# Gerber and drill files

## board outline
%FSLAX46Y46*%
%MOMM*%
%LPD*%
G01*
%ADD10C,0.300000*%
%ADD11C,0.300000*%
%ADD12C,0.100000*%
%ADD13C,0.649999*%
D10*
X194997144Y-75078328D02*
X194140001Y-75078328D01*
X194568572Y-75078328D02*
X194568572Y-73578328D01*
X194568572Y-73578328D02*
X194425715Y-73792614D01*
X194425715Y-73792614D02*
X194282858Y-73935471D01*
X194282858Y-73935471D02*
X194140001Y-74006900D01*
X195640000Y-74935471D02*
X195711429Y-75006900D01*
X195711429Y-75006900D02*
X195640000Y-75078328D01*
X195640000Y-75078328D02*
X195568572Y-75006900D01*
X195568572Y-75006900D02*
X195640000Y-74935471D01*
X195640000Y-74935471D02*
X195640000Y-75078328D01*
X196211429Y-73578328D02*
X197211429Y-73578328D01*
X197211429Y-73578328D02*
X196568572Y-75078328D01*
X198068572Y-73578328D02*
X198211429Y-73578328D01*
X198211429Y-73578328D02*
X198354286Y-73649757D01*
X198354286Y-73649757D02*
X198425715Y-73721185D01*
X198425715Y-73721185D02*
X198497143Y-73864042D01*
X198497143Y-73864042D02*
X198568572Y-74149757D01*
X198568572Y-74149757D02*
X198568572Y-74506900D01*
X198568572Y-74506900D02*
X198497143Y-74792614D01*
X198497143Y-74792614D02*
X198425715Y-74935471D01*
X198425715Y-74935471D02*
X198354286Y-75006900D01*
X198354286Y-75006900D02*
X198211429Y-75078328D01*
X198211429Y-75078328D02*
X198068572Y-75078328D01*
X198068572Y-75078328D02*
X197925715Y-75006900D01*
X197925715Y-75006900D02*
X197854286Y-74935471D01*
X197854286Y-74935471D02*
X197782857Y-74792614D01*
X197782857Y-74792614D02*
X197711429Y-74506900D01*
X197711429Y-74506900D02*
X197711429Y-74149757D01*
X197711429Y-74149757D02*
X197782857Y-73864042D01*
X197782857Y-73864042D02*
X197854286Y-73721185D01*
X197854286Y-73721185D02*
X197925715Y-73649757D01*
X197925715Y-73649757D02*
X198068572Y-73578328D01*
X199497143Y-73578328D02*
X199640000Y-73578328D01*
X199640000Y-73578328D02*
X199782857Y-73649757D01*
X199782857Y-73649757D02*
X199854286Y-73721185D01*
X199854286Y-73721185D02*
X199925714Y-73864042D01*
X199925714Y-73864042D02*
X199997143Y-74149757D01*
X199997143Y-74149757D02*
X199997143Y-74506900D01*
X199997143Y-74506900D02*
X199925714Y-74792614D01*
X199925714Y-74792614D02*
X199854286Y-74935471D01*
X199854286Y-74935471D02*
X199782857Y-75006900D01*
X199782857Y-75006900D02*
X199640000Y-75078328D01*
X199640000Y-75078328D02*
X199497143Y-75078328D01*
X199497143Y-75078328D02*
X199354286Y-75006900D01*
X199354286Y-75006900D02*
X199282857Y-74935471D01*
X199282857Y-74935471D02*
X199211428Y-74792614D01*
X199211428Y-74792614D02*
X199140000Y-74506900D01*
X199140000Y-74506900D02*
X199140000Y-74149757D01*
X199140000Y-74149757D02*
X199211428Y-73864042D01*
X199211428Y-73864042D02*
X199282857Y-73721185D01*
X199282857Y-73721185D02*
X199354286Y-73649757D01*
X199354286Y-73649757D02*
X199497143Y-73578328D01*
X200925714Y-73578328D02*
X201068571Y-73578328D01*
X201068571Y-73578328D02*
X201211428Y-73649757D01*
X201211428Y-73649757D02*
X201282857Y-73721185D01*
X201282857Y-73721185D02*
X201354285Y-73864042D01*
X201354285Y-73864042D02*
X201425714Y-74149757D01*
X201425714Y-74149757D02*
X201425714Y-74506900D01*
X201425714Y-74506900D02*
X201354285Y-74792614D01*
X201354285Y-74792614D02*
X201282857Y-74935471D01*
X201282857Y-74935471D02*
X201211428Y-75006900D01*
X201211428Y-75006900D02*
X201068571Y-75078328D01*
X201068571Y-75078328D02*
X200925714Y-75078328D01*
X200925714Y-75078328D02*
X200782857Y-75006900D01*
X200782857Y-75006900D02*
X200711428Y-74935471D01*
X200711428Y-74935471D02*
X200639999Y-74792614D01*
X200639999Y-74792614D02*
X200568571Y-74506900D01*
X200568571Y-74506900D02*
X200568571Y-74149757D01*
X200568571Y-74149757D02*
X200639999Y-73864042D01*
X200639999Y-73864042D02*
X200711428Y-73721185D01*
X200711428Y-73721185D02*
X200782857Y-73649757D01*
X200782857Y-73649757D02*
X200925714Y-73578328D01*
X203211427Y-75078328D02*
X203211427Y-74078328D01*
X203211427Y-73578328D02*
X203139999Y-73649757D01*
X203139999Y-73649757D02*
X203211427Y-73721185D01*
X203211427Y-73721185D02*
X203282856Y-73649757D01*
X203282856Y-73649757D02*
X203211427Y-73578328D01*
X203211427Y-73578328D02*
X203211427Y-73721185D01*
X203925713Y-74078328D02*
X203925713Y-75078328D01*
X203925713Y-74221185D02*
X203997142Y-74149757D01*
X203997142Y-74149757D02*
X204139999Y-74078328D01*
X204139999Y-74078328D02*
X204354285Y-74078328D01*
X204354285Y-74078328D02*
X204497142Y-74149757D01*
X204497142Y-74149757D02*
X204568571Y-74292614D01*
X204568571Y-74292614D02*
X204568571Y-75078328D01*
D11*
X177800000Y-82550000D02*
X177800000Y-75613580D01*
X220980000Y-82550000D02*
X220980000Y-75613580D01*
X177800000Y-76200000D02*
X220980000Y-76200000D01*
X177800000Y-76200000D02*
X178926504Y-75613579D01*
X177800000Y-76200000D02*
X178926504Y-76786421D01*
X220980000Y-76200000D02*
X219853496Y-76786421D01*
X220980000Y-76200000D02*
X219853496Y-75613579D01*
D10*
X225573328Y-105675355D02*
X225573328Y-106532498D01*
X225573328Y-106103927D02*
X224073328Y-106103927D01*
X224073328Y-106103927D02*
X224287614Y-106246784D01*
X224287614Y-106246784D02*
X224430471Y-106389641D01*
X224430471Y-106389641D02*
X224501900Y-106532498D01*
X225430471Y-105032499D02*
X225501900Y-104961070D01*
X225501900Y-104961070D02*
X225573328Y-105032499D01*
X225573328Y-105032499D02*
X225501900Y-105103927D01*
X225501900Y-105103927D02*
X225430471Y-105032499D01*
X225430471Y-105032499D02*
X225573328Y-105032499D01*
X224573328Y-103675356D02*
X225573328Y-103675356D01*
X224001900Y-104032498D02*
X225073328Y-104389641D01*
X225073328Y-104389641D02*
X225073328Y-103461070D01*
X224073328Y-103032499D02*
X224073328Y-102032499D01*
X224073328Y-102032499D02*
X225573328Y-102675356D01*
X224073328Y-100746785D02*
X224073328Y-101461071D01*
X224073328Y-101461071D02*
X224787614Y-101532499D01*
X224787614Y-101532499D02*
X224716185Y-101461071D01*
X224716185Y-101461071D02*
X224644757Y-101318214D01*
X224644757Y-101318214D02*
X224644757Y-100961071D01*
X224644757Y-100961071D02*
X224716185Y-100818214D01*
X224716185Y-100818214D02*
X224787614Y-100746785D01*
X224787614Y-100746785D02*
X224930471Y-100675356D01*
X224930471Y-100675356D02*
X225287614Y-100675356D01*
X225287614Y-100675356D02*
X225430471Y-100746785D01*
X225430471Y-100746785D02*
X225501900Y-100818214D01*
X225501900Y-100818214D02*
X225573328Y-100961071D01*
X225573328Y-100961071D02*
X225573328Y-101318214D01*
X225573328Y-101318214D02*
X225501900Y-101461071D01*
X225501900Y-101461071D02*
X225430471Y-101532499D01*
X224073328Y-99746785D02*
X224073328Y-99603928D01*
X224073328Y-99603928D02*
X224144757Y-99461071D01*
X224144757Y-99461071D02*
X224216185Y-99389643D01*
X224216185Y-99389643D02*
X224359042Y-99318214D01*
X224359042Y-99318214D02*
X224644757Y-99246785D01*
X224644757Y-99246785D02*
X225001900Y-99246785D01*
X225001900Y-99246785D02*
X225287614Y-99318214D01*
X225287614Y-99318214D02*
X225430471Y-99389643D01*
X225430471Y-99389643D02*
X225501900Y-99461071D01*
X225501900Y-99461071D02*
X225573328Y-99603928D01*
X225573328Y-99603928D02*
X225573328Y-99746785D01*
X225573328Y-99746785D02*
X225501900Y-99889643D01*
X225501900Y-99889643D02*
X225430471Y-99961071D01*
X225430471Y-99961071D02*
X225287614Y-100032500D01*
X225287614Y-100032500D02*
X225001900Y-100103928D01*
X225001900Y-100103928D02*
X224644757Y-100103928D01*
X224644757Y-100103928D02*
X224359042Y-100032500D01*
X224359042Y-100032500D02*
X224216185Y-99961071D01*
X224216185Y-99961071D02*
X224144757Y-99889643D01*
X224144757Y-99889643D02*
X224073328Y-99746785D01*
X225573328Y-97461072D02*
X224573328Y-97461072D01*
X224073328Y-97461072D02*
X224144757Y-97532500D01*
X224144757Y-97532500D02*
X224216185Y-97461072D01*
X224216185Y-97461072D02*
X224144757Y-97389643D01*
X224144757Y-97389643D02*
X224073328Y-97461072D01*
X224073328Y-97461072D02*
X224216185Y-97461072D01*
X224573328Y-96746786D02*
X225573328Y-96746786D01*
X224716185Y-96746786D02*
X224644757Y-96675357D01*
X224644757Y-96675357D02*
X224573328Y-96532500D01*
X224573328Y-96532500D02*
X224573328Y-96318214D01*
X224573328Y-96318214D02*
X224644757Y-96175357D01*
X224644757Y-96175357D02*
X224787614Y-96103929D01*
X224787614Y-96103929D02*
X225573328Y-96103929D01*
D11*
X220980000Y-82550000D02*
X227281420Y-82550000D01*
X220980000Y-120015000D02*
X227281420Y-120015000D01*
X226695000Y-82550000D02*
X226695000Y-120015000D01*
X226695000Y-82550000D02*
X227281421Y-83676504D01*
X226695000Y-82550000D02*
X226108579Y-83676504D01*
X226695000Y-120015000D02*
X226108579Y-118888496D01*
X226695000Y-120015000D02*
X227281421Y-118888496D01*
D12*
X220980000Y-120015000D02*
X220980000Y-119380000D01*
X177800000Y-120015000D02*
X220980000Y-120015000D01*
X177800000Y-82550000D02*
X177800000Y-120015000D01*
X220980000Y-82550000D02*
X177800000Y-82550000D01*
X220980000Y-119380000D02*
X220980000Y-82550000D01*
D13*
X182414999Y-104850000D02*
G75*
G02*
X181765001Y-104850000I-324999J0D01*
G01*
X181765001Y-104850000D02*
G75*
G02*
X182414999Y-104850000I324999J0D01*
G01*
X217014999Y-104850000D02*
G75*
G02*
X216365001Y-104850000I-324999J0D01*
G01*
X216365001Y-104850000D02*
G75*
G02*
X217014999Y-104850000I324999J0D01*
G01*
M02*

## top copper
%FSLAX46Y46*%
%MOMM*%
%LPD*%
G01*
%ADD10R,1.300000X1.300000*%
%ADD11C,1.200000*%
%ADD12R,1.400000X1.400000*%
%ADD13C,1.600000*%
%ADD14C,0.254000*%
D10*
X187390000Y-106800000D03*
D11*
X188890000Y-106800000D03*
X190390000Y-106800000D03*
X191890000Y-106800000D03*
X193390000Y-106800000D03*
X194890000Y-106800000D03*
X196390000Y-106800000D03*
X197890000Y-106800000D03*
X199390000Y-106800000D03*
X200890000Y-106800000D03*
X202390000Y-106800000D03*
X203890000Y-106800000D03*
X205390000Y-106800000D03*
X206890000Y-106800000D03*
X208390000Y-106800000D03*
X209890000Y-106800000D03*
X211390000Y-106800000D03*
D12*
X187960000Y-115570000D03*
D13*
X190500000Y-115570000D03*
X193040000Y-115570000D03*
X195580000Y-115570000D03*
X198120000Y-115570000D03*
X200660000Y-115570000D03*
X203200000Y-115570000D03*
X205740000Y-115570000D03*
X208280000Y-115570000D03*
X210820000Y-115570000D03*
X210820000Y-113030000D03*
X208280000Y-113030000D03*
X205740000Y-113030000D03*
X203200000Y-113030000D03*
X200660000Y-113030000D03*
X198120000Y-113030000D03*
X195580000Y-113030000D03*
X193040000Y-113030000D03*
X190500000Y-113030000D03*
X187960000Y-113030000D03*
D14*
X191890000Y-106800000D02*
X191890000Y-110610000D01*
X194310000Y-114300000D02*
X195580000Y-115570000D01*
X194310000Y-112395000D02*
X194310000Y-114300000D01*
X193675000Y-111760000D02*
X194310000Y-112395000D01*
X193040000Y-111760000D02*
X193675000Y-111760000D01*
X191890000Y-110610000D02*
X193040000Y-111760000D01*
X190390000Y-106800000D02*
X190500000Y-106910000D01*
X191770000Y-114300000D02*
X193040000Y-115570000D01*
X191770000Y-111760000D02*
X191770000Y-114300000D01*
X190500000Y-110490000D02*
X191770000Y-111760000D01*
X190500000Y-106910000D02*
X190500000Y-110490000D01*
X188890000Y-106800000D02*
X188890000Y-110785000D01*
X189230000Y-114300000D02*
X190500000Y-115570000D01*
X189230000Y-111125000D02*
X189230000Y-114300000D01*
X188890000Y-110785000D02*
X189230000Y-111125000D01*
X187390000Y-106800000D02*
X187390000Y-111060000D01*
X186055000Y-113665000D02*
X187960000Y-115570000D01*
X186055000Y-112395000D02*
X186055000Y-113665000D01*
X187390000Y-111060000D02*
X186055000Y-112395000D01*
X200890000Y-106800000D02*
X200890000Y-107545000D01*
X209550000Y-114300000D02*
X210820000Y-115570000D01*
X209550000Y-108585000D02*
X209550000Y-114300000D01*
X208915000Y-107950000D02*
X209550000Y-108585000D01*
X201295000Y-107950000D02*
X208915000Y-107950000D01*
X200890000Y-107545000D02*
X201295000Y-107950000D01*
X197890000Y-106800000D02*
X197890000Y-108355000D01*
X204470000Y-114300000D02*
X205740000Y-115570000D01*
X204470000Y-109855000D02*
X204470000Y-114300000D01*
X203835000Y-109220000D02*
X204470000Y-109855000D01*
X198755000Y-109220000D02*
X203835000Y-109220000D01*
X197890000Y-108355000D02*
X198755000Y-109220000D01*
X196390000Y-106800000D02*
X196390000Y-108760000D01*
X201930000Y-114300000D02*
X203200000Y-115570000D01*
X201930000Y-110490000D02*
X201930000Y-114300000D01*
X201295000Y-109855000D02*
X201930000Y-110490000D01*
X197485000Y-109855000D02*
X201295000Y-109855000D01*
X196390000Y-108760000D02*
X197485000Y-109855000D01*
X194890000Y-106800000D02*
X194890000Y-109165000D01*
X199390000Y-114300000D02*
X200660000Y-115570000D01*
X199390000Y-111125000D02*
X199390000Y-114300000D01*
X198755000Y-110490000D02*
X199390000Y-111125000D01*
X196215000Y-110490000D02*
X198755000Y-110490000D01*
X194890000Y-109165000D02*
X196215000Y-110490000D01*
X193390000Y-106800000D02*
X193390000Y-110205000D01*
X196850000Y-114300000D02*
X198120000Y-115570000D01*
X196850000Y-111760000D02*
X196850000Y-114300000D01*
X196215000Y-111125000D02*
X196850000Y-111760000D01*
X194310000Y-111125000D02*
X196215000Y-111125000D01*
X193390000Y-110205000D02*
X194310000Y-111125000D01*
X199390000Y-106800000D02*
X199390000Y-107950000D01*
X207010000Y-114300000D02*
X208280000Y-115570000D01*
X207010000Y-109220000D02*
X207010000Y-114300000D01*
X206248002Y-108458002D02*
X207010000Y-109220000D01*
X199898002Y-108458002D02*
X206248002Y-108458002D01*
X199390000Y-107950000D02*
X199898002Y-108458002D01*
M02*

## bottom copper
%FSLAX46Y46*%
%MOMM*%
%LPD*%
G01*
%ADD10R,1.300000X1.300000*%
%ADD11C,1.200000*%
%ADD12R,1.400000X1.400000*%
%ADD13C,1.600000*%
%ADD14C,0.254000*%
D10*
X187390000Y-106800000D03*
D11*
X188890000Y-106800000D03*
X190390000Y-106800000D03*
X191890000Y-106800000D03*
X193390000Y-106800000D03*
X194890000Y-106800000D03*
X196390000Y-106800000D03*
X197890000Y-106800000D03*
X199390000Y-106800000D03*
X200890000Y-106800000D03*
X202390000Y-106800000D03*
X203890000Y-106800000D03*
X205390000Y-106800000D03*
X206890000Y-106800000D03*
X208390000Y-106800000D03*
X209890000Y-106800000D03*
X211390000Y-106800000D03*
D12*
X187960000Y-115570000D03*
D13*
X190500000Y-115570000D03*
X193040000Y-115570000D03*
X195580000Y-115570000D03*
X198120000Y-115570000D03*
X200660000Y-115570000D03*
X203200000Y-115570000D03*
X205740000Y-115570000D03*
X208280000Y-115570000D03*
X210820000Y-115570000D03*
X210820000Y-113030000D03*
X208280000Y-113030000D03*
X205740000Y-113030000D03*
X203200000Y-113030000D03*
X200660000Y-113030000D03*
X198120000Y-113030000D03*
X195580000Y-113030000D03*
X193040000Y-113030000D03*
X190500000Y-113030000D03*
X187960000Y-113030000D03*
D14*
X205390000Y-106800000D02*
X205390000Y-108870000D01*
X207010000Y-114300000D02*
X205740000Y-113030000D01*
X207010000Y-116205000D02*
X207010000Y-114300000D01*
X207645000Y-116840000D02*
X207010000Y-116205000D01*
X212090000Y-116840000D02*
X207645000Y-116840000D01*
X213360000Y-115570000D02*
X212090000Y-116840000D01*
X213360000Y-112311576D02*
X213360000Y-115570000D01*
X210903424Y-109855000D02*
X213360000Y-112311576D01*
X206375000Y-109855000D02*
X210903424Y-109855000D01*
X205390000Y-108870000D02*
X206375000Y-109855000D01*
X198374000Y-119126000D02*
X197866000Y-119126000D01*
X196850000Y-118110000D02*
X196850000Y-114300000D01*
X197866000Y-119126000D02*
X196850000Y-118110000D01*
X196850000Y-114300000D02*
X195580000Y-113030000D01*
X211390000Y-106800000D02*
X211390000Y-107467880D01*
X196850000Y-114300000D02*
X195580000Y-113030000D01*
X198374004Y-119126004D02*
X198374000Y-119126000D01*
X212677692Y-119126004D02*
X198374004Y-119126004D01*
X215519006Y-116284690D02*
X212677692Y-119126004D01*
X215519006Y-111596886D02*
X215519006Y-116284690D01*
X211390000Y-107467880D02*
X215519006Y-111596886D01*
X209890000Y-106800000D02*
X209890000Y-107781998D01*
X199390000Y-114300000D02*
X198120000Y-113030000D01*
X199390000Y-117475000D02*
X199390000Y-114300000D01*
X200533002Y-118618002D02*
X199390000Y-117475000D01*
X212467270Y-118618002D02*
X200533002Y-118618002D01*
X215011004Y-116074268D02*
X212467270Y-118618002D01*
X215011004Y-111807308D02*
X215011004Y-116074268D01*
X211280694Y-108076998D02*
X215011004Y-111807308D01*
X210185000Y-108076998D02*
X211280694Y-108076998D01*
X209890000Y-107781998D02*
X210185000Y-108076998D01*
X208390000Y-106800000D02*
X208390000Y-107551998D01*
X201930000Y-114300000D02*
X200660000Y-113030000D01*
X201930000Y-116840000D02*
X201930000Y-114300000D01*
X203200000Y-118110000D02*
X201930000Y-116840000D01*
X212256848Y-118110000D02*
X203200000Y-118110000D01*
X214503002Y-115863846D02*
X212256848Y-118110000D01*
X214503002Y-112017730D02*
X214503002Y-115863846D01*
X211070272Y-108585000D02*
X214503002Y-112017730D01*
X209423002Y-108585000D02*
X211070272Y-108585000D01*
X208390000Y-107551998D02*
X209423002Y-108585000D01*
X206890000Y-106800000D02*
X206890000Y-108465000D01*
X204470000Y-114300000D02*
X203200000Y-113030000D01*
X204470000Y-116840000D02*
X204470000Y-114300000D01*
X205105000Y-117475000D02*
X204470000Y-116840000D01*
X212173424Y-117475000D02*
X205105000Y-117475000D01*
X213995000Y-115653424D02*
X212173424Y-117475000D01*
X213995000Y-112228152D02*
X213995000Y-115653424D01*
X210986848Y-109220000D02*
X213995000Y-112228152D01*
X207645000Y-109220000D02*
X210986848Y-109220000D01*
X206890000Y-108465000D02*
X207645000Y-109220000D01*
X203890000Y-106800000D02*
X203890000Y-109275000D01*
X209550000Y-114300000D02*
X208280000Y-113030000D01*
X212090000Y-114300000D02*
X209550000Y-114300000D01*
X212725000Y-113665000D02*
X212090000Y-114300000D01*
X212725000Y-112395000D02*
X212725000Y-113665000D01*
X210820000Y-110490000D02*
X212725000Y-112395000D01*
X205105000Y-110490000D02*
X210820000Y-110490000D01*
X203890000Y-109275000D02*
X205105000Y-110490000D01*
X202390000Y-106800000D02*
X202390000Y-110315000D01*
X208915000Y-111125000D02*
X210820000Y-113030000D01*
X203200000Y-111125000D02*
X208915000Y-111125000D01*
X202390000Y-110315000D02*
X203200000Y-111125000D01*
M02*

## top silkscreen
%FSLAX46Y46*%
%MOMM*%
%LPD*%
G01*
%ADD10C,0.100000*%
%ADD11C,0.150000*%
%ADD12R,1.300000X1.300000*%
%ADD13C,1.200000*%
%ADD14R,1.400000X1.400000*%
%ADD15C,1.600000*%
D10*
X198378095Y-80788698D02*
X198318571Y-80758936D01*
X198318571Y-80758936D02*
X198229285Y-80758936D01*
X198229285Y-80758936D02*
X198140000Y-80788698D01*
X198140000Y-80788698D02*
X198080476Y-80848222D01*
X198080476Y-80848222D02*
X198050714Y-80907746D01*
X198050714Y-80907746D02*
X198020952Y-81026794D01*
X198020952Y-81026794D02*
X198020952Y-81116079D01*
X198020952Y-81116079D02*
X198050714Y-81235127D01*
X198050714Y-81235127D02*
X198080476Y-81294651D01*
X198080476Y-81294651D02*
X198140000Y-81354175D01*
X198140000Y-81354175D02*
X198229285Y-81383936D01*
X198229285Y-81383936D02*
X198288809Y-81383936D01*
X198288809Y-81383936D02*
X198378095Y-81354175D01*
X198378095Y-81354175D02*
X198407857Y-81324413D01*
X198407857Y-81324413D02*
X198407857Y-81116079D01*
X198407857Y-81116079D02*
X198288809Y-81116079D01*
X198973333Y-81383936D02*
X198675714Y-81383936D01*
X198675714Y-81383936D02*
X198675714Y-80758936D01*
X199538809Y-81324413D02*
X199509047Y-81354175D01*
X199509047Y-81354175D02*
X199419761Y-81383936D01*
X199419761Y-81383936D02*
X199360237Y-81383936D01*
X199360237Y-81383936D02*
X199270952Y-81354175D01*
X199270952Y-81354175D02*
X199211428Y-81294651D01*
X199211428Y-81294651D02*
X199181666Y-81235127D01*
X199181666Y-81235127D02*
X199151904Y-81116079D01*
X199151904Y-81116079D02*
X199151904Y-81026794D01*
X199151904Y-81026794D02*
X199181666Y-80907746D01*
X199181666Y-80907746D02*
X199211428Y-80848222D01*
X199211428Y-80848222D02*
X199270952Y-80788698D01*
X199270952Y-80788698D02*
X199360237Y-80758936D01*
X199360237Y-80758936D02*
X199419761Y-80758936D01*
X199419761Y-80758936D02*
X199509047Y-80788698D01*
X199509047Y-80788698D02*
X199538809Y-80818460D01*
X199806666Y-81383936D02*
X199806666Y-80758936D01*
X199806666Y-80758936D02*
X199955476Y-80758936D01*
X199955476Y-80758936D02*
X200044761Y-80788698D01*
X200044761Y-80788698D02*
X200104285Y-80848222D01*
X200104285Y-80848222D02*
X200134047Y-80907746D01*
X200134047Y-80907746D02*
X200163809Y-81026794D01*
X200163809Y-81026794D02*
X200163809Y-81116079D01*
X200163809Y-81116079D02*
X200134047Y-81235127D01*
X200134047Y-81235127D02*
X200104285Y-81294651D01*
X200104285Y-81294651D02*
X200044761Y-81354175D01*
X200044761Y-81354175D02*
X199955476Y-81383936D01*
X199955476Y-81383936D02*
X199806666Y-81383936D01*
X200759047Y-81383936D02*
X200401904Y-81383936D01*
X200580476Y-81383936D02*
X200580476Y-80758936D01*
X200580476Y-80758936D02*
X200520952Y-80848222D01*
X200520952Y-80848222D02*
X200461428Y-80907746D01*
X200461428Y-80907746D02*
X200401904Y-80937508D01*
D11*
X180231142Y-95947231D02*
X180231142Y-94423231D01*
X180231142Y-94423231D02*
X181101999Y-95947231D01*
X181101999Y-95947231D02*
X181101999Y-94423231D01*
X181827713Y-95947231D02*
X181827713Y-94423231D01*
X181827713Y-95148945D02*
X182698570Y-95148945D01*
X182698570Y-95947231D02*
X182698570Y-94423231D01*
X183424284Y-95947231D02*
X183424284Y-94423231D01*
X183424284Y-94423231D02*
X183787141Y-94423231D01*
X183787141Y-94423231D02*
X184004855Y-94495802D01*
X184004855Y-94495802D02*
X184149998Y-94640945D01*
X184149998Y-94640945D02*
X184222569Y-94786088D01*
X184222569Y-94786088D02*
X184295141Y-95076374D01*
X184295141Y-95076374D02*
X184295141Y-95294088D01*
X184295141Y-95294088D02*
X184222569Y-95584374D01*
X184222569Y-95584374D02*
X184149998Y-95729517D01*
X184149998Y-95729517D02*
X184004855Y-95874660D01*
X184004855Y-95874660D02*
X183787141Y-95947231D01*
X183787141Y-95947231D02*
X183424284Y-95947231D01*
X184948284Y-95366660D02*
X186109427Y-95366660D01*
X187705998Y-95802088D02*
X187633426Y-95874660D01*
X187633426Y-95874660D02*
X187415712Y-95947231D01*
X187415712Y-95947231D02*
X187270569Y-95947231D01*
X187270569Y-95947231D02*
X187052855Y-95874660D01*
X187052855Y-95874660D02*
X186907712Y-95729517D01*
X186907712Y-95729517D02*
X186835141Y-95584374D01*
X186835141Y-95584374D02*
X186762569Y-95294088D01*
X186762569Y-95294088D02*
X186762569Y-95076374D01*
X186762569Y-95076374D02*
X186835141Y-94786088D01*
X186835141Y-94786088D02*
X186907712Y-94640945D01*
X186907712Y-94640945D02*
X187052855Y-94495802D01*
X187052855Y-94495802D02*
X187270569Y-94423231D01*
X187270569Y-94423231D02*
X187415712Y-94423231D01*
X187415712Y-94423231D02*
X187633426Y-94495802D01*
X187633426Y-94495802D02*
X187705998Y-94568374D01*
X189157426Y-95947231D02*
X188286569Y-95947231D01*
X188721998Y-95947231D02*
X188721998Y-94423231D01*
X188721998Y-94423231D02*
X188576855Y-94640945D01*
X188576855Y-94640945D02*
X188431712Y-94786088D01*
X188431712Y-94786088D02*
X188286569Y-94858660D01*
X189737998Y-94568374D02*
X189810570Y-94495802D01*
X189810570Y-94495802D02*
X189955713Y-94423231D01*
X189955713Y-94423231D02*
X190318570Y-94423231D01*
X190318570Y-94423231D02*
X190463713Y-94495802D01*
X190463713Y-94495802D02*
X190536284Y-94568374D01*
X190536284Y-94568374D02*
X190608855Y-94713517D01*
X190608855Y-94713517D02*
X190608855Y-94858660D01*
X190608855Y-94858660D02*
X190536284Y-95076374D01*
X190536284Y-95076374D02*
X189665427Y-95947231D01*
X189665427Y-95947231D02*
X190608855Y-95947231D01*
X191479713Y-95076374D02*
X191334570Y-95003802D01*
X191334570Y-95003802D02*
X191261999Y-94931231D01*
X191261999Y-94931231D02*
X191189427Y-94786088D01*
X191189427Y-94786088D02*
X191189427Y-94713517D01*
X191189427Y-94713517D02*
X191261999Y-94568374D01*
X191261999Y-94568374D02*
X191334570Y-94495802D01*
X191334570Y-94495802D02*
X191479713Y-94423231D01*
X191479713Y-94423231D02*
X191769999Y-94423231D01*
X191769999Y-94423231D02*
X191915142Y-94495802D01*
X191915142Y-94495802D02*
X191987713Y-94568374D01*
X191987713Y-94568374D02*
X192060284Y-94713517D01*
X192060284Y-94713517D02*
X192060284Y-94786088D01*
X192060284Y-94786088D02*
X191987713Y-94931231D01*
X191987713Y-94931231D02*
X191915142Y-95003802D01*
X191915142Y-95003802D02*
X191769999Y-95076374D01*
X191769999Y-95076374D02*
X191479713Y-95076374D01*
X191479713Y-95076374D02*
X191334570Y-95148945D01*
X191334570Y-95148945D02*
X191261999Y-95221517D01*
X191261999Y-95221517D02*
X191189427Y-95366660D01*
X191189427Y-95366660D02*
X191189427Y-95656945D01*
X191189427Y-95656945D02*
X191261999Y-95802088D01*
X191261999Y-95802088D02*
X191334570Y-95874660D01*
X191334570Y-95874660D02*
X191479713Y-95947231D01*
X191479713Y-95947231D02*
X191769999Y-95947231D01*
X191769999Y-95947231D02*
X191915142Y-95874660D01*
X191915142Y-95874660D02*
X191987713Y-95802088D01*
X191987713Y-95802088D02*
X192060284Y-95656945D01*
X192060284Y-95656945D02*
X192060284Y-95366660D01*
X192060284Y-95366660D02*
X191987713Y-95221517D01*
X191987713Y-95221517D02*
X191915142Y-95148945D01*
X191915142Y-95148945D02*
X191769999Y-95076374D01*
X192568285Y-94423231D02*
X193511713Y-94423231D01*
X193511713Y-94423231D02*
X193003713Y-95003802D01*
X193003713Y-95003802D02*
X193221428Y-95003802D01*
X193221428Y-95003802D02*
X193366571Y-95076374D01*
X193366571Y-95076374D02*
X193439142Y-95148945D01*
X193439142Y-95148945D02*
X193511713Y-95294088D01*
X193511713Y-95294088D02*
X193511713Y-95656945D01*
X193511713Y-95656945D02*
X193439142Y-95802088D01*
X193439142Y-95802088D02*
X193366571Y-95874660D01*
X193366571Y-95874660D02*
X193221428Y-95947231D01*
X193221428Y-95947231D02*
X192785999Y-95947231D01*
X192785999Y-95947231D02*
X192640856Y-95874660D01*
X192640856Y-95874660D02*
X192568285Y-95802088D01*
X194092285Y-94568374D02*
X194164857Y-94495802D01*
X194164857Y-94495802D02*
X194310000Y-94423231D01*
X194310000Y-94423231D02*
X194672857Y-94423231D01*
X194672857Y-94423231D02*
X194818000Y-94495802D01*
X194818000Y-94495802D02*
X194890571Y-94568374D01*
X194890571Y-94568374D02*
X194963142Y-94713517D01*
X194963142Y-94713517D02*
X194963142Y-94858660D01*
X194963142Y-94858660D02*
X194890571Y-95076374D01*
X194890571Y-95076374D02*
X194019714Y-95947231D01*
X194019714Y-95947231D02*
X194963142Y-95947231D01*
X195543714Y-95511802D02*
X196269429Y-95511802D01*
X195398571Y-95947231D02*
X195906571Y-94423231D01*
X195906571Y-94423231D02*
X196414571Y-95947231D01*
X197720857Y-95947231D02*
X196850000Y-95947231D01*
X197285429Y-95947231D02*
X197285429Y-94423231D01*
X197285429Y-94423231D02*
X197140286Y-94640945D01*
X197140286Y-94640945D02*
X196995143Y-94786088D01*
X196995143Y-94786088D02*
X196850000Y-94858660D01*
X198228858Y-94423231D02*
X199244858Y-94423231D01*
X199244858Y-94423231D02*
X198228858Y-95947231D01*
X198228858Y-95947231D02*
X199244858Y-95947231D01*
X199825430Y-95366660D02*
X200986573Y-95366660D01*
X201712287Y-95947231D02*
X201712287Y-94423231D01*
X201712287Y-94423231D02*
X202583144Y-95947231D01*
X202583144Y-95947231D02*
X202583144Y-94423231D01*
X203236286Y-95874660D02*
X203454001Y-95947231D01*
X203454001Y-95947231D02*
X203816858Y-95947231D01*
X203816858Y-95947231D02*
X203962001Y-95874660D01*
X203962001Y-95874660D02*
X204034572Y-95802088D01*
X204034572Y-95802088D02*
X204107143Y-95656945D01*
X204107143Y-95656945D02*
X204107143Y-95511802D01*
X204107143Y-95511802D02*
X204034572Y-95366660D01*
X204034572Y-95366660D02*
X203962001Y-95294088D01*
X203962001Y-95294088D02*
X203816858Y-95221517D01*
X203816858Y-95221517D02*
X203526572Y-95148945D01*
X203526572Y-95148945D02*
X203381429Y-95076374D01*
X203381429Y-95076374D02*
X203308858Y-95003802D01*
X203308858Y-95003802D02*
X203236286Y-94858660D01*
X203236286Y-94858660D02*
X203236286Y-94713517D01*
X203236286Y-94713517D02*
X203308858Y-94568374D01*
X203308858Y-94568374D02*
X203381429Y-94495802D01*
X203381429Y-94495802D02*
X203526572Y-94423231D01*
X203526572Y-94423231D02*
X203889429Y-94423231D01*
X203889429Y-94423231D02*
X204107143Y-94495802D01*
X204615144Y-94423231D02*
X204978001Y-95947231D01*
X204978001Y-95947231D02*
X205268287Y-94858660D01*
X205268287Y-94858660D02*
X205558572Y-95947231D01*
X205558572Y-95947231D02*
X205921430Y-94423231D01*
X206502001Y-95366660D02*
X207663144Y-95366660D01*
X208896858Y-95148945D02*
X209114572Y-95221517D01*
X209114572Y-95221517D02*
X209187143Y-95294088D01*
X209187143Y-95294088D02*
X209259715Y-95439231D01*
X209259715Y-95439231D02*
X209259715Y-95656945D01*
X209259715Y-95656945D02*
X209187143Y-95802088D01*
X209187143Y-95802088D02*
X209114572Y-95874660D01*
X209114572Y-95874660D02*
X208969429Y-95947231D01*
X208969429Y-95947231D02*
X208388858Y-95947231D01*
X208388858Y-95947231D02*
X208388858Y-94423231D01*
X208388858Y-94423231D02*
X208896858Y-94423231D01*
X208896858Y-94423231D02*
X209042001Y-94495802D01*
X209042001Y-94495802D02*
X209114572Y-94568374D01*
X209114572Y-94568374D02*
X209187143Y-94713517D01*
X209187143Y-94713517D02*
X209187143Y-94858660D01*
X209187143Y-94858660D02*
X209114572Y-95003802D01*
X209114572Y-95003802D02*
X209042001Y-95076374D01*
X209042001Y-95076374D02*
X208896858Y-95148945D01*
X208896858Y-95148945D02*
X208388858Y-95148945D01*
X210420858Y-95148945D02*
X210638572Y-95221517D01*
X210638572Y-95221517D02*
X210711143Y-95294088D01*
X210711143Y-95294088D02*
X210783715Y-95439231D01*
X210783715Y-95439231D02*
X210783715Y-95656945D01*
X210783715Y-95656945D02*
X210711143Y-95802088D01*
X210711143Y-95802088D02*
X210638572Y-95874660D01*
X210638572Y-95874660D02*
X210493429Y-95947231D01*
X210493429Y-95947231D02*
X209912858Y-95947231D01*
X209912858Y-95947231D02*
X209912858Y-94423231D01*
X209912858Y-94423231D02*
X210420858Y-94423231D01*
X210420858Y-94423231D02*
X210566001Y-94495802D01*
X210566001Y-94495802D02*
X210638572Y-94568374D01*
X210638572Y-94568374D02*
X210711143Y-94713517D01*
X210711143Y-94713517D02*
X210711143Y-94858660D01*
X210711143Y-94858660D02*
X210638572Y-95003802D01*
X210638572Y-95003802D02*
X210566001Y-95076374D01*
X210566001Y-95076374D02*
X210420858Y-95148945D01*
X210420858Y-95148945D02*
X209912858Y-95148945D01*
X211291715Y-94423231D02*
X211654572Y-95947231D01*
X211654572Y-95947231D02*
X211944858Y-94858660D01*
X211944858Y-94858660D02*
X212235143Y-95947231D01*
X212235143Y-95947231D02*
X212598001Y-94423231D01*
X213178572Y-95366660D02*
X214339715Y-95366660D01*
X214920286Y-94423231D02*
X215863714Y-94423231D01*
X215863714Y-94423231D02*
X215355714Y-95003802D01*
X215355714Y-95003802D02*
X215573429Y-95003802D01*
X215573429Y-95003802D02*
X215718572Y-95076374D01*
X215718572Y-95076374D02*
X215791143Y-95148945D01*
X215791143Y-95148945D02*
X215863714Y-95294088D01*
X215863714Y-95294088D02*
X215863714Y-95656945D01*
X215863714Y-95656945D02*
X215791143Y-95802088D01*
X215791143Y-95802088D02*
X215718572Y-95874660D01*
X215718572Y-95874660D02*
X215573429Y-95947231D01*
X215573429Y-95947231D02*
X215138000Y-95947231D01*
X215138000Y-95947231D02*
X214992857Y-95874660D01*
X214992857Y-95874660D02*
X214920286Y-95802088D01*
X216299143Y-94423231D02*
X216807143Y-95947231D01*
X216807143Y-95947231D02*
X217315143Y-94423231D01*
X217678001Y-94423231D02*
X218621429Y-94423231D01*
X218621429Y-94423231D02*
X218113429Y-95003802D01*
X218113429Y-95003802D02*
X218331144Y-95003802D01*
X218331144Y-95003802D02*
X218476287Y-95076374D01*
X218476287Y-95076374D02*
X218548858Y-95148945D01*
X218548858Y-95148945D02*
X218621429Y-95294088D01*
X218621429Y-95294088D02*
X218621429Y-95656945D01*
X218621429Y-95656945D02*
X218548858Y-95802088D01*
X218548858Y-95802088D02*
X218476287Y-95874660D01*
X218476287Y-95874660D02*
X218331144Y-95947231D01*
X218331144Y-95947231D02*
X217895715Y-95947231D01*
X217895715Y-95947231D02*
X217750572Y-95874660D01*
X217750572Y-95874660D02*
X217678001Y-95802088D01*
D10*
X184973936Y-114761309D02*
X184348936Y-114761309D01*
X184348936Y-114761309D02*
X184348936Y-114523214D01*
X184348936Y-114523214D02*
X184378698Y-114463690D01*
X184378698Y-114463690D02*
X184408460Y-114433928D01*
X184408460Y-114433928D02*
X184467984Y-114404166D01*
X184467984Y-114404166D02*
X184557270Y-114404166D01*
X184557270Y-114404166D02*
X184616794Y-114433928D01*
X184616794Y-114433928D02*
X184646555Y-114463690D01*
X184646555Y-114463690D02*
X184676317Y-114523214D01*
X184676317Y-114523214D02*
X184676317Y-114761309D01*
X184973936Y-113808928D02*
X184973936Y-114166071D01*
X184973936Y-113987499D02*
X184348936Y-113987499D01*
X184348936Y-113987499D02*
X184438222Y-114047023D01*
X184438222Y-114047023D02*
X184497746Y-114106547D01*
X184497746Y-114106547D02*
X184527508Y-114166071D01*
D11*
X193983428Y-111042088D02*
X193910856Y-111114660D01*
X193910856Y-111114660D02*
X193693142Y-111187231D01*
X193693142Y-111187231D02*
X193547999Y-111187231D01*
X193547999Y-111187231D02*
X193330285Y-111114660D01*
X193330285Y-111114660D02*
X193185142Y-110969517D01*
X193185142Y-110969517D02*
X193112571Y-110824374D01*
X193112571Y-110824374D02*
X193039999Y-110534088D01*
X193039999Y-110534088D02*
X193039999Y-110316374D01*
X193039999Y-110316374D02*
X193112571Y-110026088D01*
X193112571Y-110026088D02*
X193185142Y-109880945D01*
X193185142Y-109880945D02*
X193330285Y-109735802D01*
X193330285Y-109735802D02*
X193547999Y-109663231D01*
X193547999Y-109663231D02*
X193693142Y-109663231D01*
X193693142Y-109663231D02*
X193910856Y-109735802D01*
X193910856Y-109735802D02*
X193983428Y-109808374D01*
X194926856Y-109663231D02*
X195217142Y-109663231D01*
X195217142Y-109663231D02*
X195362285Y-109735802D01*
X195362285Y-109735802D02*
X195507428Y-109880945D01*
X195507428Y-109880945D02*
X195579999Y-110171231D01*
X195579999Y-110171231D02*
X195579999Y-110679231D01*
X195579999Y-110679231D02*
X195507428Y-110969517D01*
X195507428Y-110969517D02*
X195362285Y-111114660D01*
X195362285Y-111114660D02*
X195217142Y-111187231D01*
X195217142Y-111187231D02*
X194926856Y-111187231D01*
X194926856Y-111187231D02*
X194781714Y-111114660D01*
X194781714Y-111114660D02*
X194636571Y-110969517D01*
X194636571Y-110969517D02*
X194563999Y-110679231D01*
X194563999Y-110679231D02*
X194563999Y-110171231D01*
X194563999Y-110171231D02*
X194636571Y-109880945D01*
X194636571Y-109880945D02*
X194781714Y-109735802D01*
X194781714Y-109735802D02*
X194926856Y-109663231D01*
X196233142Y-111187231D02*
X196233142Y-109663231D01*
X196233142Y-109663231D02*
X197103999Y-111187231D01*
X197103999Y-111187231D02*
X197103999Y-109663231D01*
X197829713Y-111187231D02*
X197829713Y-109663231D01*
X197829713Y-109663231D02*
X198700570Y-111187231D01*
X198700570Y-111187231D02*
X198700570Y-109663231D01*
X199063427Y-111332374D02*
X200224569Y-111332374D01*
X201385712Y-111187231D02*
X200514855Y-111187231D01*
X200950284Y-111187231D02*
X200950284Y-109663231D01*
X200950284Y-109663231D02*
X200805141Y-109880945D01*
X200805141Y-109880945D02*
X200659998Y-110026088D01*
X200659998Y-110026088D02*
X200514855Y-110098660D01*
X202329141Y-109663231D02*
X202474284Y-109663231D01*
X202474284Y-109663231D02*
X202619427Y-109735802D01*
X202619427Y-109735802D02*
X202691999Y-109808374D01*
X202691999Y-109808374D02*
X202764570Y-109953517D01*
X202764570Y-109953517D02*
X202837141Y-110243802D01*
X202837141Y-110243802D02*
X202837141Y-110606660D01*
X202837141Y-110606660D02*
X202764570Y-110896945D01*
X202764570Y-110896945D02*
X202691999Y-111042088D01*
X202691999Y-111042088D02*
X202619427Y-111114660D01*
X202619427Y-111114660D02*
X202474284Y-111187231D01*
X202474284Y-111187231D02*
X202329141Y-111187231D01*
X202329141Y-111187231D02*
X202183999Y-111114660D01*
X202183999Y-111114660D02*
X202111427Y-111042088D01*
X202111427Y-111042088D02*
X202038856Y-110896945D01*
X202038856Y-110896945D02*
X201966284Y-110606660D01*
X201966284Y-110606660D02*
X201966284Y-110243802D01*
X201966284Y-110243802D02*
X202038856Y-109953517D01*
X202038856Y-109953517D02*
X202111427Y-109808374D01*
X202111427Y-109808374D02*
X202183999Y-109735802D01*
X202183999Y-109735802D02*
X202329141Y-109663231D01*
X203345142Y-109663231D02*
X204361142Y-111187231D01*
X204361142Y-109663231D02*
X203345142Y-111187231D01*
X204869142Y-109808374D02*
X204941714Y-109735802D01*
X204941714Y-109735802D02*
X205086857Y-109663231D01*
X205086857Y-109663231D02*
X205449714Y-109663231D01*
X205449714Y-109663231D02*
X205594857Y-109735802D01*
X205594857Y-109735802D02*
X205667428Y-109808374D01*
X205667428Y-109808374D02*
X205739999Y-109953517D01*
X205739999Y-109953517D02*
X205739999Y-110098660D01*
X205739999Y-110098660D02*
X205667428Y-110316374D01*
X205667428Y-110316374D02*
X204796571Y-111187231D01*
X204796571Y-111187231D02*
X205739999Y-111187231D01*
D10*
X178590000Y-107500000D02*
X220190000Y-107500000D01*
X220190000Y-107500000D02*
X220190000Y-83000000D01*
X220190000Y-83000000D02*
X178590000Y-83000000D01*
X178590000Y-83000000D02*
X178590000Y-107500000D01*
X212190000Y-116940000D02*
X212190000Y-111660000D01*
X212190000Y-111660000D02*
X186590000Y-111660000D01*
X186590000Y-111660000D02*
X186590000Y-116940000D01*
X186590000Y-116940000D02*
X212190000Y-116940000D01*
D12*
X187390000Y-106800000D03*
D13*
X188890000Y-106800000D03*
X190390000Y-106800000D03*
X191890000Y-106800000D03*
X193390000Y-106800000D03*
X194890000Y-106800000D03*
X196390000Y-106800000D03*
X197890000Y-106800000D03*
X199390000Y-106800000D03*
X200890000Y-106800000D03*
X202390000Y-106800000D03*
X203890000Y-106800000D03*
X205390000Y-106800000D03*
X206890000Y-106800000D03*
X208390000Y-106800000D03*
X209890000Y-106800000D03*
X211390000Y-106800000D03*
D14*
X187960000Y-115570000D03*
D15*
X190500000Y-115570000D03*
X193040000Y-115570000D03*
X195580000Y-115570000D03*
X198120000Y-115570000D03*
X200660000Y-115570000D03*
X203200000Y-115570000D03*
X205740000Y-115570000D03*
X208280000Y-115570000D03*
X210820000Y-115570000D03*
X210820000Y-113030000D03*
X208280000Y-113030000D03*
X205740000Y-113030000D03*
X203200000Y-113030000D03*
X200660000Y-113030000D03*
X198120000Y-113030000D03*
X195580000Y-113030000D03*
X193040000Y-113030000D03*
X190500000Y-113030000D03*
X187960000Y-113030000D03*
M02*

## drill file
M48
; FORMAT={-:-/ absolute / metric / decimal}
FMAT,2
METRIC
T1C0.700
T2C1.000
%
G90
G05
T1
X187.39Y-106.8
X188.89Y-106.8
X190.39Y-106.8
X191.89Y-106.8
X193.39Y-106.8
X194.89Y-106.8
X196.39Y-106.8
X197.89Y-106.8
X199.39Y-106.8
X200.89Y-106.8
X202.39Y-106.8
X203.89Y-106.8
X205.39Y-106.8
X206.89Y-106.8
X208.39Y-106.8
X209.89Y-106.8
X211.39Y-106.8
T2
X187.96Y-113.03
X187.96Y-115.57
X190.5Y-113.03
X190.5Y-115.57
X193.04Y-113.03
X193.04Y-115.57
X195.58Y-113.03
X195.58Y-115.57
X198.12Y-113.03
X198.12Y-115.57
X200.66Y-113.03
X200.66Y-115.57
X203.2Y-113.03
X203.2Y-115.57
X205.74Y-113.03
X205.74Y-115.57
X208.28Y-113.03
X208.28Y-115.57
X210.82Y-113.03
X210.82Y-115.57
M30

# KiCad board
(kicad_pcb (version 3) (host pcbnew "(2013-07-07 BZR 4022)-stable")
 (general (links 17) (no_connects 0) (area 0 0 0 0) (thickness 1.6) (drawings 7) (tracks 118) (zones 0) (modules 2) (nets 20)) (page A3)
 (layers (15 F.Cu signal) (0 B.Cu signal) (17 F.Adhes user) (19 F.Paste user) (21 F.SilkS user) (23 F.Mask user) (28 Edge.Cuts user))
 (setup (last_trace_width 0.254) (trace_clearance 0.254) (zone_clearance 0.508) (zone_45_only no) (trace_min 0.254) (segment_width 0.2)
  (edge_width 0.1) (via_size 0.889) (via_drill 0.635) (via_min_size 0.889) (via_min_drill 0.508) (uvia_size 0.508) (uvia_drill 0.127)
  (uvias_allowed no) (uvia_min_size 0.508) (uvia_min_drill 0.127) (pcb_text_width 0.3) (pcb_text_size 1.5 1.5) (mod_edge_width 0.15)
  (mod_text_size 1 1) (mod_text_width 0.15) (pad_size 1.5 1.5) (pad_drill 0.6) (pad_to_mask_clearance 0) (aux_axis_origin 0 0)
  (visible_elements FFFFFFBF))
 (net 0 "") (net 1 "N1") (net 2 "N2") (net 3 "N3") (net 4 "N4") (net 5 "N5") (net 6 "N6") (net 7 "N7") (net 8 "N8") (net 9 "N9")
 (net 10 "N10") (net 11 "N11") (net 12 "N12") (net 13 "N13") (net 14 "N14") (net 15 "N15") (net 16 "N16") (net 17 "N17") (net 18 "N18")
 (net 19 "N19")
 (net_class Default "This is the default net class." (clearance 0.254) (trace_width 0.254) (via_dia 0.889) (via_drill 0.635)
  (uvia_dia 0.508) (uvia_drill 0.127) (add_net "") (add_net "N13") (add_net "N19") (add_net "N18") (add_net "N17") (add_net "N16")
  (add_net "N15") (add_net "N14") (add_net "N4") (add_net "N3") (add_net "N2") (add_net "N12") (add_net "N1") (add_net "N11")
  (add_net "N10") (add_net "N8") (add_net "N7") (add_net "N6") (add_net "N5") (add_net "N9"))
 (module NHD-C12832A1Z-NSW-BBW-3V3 (layer F.Cu) (at 199.39 95.25)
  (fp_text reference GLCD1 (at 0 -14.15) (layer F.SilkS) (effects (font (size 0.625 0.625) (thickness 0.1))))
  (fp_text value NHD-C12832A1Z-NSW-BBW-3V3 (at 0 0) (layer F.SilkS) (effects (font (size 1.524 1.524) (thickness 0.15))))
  (fp_line (start -20.8 12.25) (end 20.8 12.25) (layer F.SilkS) (width 0.1))
  (fp_line (start 20.8 12.25) (end 20.8 -12.25) (layer F.SilkS) (width 0.1))
  (fp_line (start 20.8 -12.25) (end -20.8 -12.25) (layer F.SilkS) (width 0.1))
  (fp_line (start -20.8 -12.25) (end -20.8 12.25) (layer F.SilkS) (width 0.1))
  (fp_circle (center -17.3 9.6) (end -16.840381 10.059619) (layer Edge.Cuts))
  (fp_circle (center 17.3 9.6) (end 17.759619 10.059619) (layer Edge.Cuts))
  (pad 1 thru_hole rect (at -12 11.55) (size 1.3 1.3) (drill 0.7) (layers *.Cu *.Mask F.SilkS) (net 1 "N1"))
  (pad 2 thru_hole circle (at -10.5 11.55) (size 1.2 1.2) (drill 0.7) (layers *.Cu *.Mask F.SilkS) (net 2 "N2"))
  (pad 3 thru_hole circle (at -9 11.55) (size 1.2 1.2) (drill 0.7) (layers *.Cu *.Mask F.SilkS) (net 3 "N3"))
  (pad 4 thru_hole circle (at -7.5 11.55) (size 1.2 1.2) (drill 0.7) (layers *.Cu *.Mask F.SilkS) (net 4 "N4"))
  (pad 5 thru_hole circle (at -6 11.55) (size 1.2 1.2) (drill 0.7) (layers *.Cu *.Mask F.SilkS) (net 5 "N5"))
  (pad 6 thru_hole circle (at -4.5 11.55) (size 1.2 1.2) (drill 0.7) (layers *.Cu *.Mask F.SilkS) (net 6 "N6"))
  (pad 7 thru_hole circle (at -3 11.55) (size 1.2 1.2) (drill 0.7) (layers *.Cu *.Mask F.SilkS) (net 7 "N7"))
  (pad 8 thru_hole circle (at -1.5 11.55) (size 1.2 1.2) (drill 0.7) (layers *.Cu *.Mask F.SilkS) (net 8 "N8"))
  (pad 9 thru_hole circle (at 0 11.55) (size 1.2 1.2) (drill 0.7) (layers *.Cu *.Mask F.SilkS) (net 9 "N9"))
  (pad 10 thru_hole circle (at 1.5 11.55) (size 1.2 1.2) (drill 0.7) (layers *.Cu *.Mask F.SilkS) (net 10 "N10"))
  (pad 11 thru_hole circle (at 3 11.55) (size 1.2 1.2) (drill 0.7) (layers *.Cu *.Mask F.SilkS) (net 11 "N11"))
  (pad 12 thru_hole circle (at 4.5 11.55) (size 1.2 1.2) (drill 0.7) (layers *.Cu *.Mask F.SilkS) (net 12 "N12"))
  (pad 13 thru_hole circle (at 6 11.55) (size 1.2 1.2) (drill 0.7) (layers *.Cu *.Mask F.SilkS) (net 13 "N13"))
  (pad 14 thru_hole circle (at 7.5 11.55) (size 1.2 1.2) (drill 0.7) (layers *.Cu *.Mask F.SilkS) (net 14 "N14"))
  (pad 15 thru_hole circle (at 9 11.55) (size 1.2 1.2) (drill 0.7) (layers *.Cu *.Mask F.SilkS) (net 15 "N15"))
  (pad 16 thru_hole circle (at 10.5 11.55) (size 1.2 1.2) (drill 0.7) (layers *.Cu *.Mask F.SilkS) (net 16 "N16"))
  (pad 17 thru_hole circle (at 12 11.55) (size 1.2 1.2) (drill 0.7) (layers *.Cu *.Mask F.SilkS) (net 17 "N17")))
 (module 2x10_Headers (layer F.Cu) (at 199.39 114.3 90)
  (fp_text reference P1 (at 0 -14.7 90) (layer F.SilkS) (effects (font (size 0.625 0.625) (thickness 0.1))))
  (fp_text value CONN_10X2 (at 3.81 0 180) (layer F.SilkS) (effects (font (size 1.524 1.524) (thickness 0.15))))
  (fp_line (start -2.64 12.8) (end 2.64 12.8) (layer F.SilkS) (width 0.1))
  (fp_line (start 2.64 12.8) (end 2.64 -12.8) (layer F.SilkS) (width 0.1))
  (fp_line (start 2.64 -12.8) (end -2.64 -12.8) (layer F.SilkS) (width 0.1))
  (fp_line (start -2.64 -12.8) (end -2.64 12.8) (layer F.SilkS) (width 0.1))
  (pad 1 thru_hole rect (at -1.27 -11.43 90) (size 1.4 1.4) (drill 1) (layers *.Cu *.Mask F.SilkS) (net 1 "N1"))
  (pad 2 thru_hole circle (at -1.27 -8.89 90) (size 1.6 1.6) (drill 1) (layers *.Cu *.Mask F.SilkS) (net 2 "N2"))
  (pad 3 thru_hole circle (at -1.27 -6.35 90) (size 1.6 1.6) (drill 1) (layers *.Cu *.Mask F.SilkS) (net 3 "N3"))
  (pad 4 thru_hole circle (at -1.27 -3.81 90) (size 1.6 1.6) (drill 1) (layers *.Cu *.Mask F.SilkS) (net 4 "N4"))
  (pad 5 thru_hole circle (at -1.27 -1.27 90) (size 1.6 1.6) (drill 1) (layers *.Cu *.Mask F.SilkS) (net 5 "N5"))
  (pad 6 thru_hole circle (at -1.27 1.27 90) (size 1.6 1.6) (drill 1) (layers *.Cu *.Mask F.SilkS) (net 6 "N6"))
  (pad 7 thru_hole circle (at -1.27 3.81 90) (size 1.6 1.6) (drill 1) (layers *.Cu *.Mask F.SilkS) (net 7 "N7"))
  (pad 8 thru_hole circle (at -1.27 6.35 90) (size 1.6 1.6) (drill 1) (layers *.Cu *.Mask F.SilkS) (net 8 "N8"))
  (pad 9 thru_hole circle (at -1.27 8.89 90) (size 1.6 1.6) (drill 1) (layers *.Cu *.Mask F.SilkS) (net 9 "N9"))
  (pad 10 thru_hole circle (at -1.27 11.43 90) (size 1.6 1.6) (drill 1) (layers *.Cu *.Mask F.SilkS) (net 10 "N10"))
  (pad 11 thru_hole circle (at 1.27 11.43 90) (size 1.6 1.6) (drill 1) (layers *.Cu *.Mask F.SilkS) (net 11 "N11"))
  (pad 12 thru_hole circle (at 1.27 8.89 90) (size 1.6 1.6) (drill 1) (layers *.Cu *.Mask F.SilkS) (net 12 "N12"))
  (pad 13 thru_hole circle (at 1.27 6.35 90) (size 1.6 1.6) (drill 1) (layers *.Cu *.Mask F.SilkS) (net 13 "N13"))
  (pad 14 thru_hole circle (at 1.27 3.81 90) (size 1.6 1.6) (drill 1) (layers *.Cu *.Mask F.SilkS) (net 14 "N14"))
  (pad 15 thru_hole circle (at 1.27 1.27 90) (size 1.6 1.6) (drill 1) (layers *.Cu *.Mask F.SilkS) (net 15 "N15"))
  (pad 16 thru_hole circle (at 1.27 -1.27 90) (size 1.6 1.6) (drill 1) (layers *.Cu *.Mask F.SilkS) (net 16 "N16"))
  (pad 17 thru_hole circle (at 1.27 -3.81 90) (size 1.6 1.6) (drill 1) (layers *.Cu *.Mask F.SilkS) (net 17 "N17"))
  (pad 18 thru_hole circle (at 1.27 -6.35 90) (size 1.6 1.6) (drill 1) (layers *.Cu *.Mask F.SilkS) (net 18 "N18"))
  (pad 19 thru_hole circle (at 1.27 -8.89 90) (size 1.6 1.6) (drill 1) (layers *.Cu *.Mask F.SilkS) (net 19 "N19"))
  (pad 20 thru_hole circle (at 1.27 -11.43 90) (size 1.6 1.6) (drill 1) (layers *.Cu *.Mask F.SilkS)))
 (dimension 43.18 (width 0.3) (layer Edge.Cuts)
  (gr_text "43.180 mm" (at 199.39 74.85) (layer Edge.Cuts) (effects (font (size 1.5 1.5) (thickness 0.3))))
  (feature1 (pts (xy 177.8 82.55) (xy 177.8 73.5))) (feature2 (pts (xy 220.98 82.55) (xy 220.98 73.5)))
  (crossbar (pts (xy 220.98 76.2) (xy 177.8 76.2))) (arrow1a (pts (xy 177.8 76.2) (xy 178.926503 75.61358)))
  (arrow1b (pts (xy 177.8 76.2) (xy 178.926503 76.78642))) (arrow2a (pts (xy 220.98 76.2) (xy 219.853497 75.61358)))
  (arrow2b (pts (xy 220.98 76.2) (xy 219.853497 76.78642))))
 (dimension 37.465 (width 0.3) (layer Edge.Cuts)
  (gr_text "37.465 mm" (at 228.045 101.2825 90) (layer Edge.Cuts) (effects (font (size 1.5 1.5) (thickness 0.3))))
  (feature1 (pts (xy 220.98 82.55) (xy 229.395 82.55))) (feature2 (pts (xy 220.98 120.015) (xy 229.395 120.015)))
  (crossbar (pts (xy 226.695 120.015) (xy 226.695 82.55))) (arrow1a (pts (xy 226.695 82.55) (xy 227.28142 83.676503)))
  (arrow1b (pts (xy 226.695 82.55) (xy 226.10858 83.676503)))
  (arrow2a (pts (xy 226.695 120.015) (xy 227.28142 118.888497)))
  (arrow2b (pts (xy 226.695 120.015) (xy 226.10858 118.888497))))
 (gr_line (start 220.98 120.015) (end 220.98 119.38) (angle 90) (layer Edge.Cuts) (width 0.1))
 (gr_line (start 177.8 120.015) (end 220.98 120.015) (angle 90) (layer Edge.Cuts) (width 0.1))
 (gr_line (start 177.8 82.55) (end 177.8 120.015) (angle 90) (layer Edge.Cuts) (width 0.1))
 (gr_line (start 220.98 82.55) (end 177.8 82.55) (angle 90) (layer Edge.Cuts) (width 0.1))
 (gr_line (start 220.98 119.38) (end 220.98 82.55) (angle 90) (layer Edge.Cuts) (width 0.1))
 (segment (start 205.39 106.8) (end 205.39 108.87) (width 0.254) (layer B.Cu) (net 13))
 (segment (start 207.01 114.3) (end 205.74 113.03) (width 0.254) (layer B.Cu) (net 13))
 (segment (start 207.01 116.205) (end 207.01 114.3) (width 0.254) (layer B.Cu) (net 13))
 (segment (start 207.645 116.84) (end 207.01 116.205) (width 0.254) (layer B.Cu) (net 13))
 (segment (start 212.09 116.84) (end 207.645 116.84) (width 0.254) (layer B.Cu) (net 13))
 (segment (start 213.36 115.57) (end 212.09 116.84) (width 0.254) (layer B.Cu) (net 13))
 (segment (start 213.36 112.311576) (end 213.36 115.57) (width 0.254) (layer B.Cu) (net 13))
 (segment (start 210.903424 109.855) (end 213.36 112.311576) (width 0.254) (layer B.Cu) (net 13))
 (segment (start 206.375 109.855) (end 210.903424 109.855) (width 0.254) (layer B.Cu) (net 13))
 (segment (start 205.39 108.87) (end 206.375 109.855) (width 0.254) (layer B.Cu) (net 13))
 (segment (start 198.374 119.126) (end 197.866 119.126) (width 0.254) (layer B.Cu) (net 17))
 (segment (start 196.85 118.11) (end 196.85 114.3) (width 0.254) (layer B.Cu) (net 17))
 (segment (start 197.866 119.126) (end 196.85 118.11) (width 0.254) (layer B.Cu) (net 17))
 (segment (start 196.85 114.3) (end 195.58 113.03) (width 0.254) (layer B.Cu) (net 17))
 (segment (start 211.39 106.8) (end 211.39 107.46788) (width 0.254) (layer B.Cu) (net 17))
 (segment (start 196.85 114.3) (end 195.58 113.03) (width 0.254) (layer B.Cu) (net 17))
 (segment (start 198.374004 119.126004) (end 198.374 119.126) (width 0.254) (layer B.Cu) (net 17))
 (segment (start 212.677692 119.126004) (end 198.374004 119.126004) (width 0.254) (layer B.Cu) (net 17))
 (segment (start 215.519006 116.28469) (end 212.677692 119.126004) (width 0.254) (layer B.Cu) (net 17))
 (segment (start 215.519006 111.596886) (end 215.519006 116.28469) (width 0.254) (layer B.Cu) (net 17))
 (segment (start 211.39 107.46788) (end 215.519006 111.596886) (width 0.254) (layer B.Cu) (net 17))
 (segment (start 209.89 106.8) (end 209.89 107.781998) (width 0.254) (layer B.Cu) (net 16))
 (segment (start 199.39 114.3) (end 198.12 113.03) (width 0.254) (layer B.Cu) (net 16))
 (segment (start 199.39 117.475) (end 199.39 114.3) (width 0.254) (layer B.Cu) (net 16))
 (segment (start 200.533002 118.618002) (end 199.39 117.475) (width 0.254) (layer B.Cu) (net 16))
 (segment (start 212.46727 118.618002) (end 200.533002 118.618002) (width 0.254) (layer B.Cu) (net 16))
 (segment (start 215.011004 116.074268) (end 212.46727 118.618002) (width 0.254) (layer B.Cu) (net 16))
 (segment (start 215.011004 111.807308) (end 215.011004 116.074268) (width 0.254) (layer B.Cu) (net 16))
 (segment (start 211.280694 108.076998) (end 215.011004 111.807308) (width 0.254) (layer B.Cu) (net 16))
 (segment (start 210.185 108.076998) (end 211.280694 108.076998) (width 0.254) (layer B.Cu) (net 16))
 (segment (start 209.89 107.781998) (end 210.185 108.076998) (width 0.254) (layer B.Cu) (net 16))
 (segment (start 208.39 106.8) (end 208.39 107.551998) (width 0.254) (layer B.Cu) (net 15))
 (segment (start 201.93 114.3) (end 200.66 113.03) (width 0.254) (layer B.Cu) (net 15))
 (segment (start 201.93 116.84) (end 201.93 114.3) (width 0.254) (layer B.Cu) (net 15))
 (segment (start 203.2 118.11) (end 201.93 116.84) (width 0.254) (layer B.Cu) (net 15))
 (segment (start 212.256848 118.11) (end 203.2 118.11) (width 0.254) (layer B.Cu) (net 15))
 (segment (start 214.503002 115.863846) (end 212.256848 118.11) (width 0.254) (layer B.Cu) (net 15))
 (segment (start 214.503002 112.01773) (end 214.503002 115.863846) (width 0.254) (layer B.Cu) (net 15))
 (segment (start 211.070272 108.585) (end 214.503002 112.01773) (width 0.254) (layer B.Cu) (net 15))
 (segment (start 209.423002 108.585) (end 211.070272 108.585) (width 0.254) (layer B.Cu) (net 15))
 (segment (start 208.39 107.551998) (end 209.423002 108.585) (width 0.254) (layer B.Cu) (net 15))
 (segment (start 206.89 106.8) (end 206.89 108.465) (width 0.254) (layer B.Cu) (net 14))
 (segment (start 204.47 114.3) (end 203.2 113.03) (width 0.254) (layer B.Cu) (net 14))
 (segment (start 204.47 116.84) (end 204.47 114.3) (width 0.254) (layer B.Cu) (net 14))
 (segment (start 205.105 117.475) (end 204.47 116.84) (width 0.254) (layer B.Cu) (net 14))
 (segment (start 212.173424 117.475) (end 205.105 117.475) (width 0.254) (layer B.Cu) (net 14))
 (segment (start 213.995 115.653424) (end 212.173424 117.475) (width 0.254) (layer B.Cu) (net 14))
 (segment (start 213.995 112.228152) (end 213.995 115.653424) (width 0.254) (layer B.Cu) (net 14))
 (segment (start 210.986848 109.22) (end 213.995 112.228152) (width 0.254) (layer B.Cu) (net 14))
 (segment (start 207.645 109.22) (end 210.986848 109.22) (width 0.254) (layer B.Cu) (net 14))
 (segment (start 206.89 108.465) (end 207.645 109.22) (width 0.254) (layer B.Cu) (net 14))
 (segment (start 191.89 106.8) (end 191.89 110.61) (width 0.254) (layer F.Cu) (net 4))
 (segment (start 194.31 114.3) (end 195.58 115.57) (width 0.254) (layer F.Cu) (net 4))
 (segment (start 194.31 112.395) (end 194.31 114.3) (width 0.254) (layer F.Cu) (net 4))
 (segment (start 193.675 111.76) (end 194.31 112.395) (width 0.254) (layer F.Cu) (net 4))
 (segment (start 193.04 111.76) (end 193.675 111.76) (width 0.254) (layer F.Cu) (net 4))
 (segment (start 191.89 110.61) (end 193.04 111.76) (width 0.254) (layer F.Cu) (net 4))
 (segment (start 190.39 106.8) (end 190.5 106.91) (width 0.254) (layer F.Cu) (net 3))
 (segment (start 191.77 114.3) (end 193.04 115.57) (width 0.254) (layer F.Cu) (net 3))
 (segment (start 191.77 111.76) (end 191.77 114.3) (width 0.254) (layer F.Cu) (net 3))
 (segment (start 190.5 110.49) (end 191.77 111.76) (width 0.254) (layer F.Cu) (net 3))
 (segment (start 190.5 106.91) (end 190.5 110.49) (width 0.254) (layer F.Cu) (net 3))
 (segment (start 188.89 106.8) (end 188.89 110.785) (width 0.254) (layer F.Cu) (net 2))
 (segment (start 189.23 114.3) (end 190.5 115.57) (width 0.254) (layer F.Cu) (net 2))
 (segment (start 189.23 111.125) (end 189.23 114.3) (width 0.254) (layer F.Cu) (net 2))
 (segment (start 188.89 110.785) (end 189.23 111.125) (width 0.254) (layer F.Cu) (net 2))
 (segment (start 203.89 106.8) (end 203.89 109.275) (width 0.254) (layer B.Cu) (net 12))
 (segment (start 209.55 114.3) (end 208.28 113.03) (width 0.254) (layer B.Cu) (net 12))
 (segment (start 212.09 114.3) (end 209.55 114.3) (width 0.254) (layer B.Cu) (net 12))
 (segment (start 212.725 113.665) (end 212.09 114.3) (width 0.254) (layer B.Cu) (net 12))
 (segment (start 212.725 112.395) (end 212.725 113.665) (width 0.254) (layer B.Cu) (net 12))
 (segment (start 210.82 110.49) (end 212.725 112.395) (width 0.254) (layer B.Cu) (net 12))
 (segment (start 205.105 110.49) (end 210.82 110.49) (width 0.254) (layer B.Cu) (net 12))
 (segment (start 203.89 109.275) (end 205.105 110.49) (width 0.254) (layer B.Cu) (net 12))
 (segment (start 187.39 106.8) (end 187.39 111.06) (width 0.254) (layer F.Cu) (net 1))
 (segment (start 186.055 113.665) (end 187.96 115.57) (width 0.254) (layer F.Cu) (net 1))
 (segment (start 186.055 112.395) (end 186.055 113.665) (width 0.254) (layer F.Cu) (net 1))
 (segment (start 187.39 111.06) (end 186.055 112.395) (width 0.254) (layer F.Cu) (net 1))
 (segment (start 202.39 106.8) (end 202.39 110.315) (width 0.254) (layer B.Cu) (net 11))
 (segment (start 208.915 111.125) (end 210.82 113.03) (width 0.254) (layer B.Cu) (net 11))
 (segment (start 203.2 111.125) (end 208.915 111.125) (width 0.254) (layer B.Cu) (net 11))
 (segment (start 202.39 110.315) (end 203.2 111.125) (width 0.254) (layer B.Cu) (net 11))
 (segment (start 200.89 106.8) (end 200.89 107.545) (width 0.254) (layer F.Cu) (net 10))
 (segment (start 209.55 114.3) (end 210.82 115.57) (width 0.254) (layer F.Cu) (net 10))
 (segment (start 209.55 108.585) (end 209.55 114.3) (width 0.254) (layer F.Cu) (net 10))
 (segment (start 208.915 107.95) (end 209.55 108.585) (width 0.254) (layer F.Cu) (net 10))
 (segment (start 201.295 107.95) (end 208.915 107.95) (width 0.254) (layer F.Cu) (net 10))
 (segment (start 200.89 107.545) (end 201.295 107.95) (width 0.254) (layer F.Cu) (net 10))
 (segment (start 197.89 106.8) (end 197.89 108.355) (width 0.254) (layer F.Cu) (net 8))
 (segment (start 204.47 114.3) (end 205.74 115.57) (width 0.254) (layer F.Cu) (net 8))
 (segment (start 204.47 109.855) (end 204.47 114.3) (width 0.254) (layer F.Cu) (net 8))
 (segment (start 203.835 109.22) (end 204.47 109.855) (width 0.254) (layer F.Cu) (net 8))
 (segment (start 198.755 109.22) (end 203.835 109.22) (width 0.254) (layer F.Cu) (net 8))
 (segment (start 197.89 108.355) (end 198.755 109.22) (width 0.254) (layer F.Cu) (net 8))
 (segment (start 196.39 106.8) (end 196.39 108.76) (width 0.254) (layer F.Cu) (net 7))
 (segment (start 201.93 114.3) (end 203.2 115.57) (width 0.254) (layer F.Cu) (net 7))
 (segment (start 201.93 110.49) (end 201.93 114.3) (width 0.254) (layer F.Cu) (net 7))
 (segment (start 201.295 109.855) (end 201.93 110.49) (width 0.254) (layer F.Cu) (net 7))
 (segment (start 197.485 109.855) (end 201.295 109.855) (width 0.254) (layer F.Cu) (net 7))
 (segment (start 196.39 108.76) (end 197.485 109.855) (width 0.254) (layer F.Cu) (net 7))
 (segment (start 194.89 106.8) (end 194.89 109.165) (width 0.254) (layer F.Cu) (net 6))
 (segment (start 199.39 114.3) (end 200.66 115.57) (width 0.254) (layer F.Cu) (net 6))
 (segment (start 199.39 111.125) (end 199.39 114.3) (width 0.254) (layer F.Cu) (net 6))
 (segment (start 198.755 110.49) (end 199.39 111.125) (width 0.254) (layer F.Cu) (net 6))
 (segment (start 196.215 110.49) (end 198.755 110.49) (width 0.254) (layer F.Cu) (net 6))
 (segment (start 194.89 109.165) (end 196.215 110.49) (width 0.254) (layer F.Cu) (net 6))
 (segment (start 193.39 106.8) (end 193.39 110.205) (width 0.254) (layer F.Cu) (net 5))
 (segment (start 196.85 114.3) (end 198.12 115.57) (width 0.254) (layer F.Cu) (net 5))
 (segment (start 196.85 111.76) (end 196.85 114.3) (width 0.254) (layer F.Cu) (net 5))
 (segment (start 196.215 111.125) (end 196.85 111.76) (width 0.254) (layer F.Cu) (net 5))
 (segment (start 194.31 111.125) (end 196.215 111.125) (width 0.254) (layer F.Cu) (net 5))
 (segment (start 193.39 110.205) (end 194.31 111.125) (width 0.254) (layer F.Cu) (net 5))
 (segment (start 199.39 106.8) (end 199.39 107.95) (width 0.254) (layer F.Cu) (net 9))
 (segment (start 207.01 114.3) (end 208.28 115.57) (width 0.254) (layer F.Cu) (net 9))
 (segment (start 207.01 109.22) (end 207.01 114.3) (width 0.254) (layer F.Cu) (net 9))
 (segment (start 206.248002 108.458002) (end 207.01 109.22) (width 0.254) (layer F.Cu) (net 9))
 (segment (start 199.898002 108.458002) (end 206.248002 108.458002) (width 0.254) (layer F.Cu) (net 9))
 (segment (start 199.39 107.95) (end 199.898002 108.458002) (width 0.254) (layer F.Cu) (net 9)))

